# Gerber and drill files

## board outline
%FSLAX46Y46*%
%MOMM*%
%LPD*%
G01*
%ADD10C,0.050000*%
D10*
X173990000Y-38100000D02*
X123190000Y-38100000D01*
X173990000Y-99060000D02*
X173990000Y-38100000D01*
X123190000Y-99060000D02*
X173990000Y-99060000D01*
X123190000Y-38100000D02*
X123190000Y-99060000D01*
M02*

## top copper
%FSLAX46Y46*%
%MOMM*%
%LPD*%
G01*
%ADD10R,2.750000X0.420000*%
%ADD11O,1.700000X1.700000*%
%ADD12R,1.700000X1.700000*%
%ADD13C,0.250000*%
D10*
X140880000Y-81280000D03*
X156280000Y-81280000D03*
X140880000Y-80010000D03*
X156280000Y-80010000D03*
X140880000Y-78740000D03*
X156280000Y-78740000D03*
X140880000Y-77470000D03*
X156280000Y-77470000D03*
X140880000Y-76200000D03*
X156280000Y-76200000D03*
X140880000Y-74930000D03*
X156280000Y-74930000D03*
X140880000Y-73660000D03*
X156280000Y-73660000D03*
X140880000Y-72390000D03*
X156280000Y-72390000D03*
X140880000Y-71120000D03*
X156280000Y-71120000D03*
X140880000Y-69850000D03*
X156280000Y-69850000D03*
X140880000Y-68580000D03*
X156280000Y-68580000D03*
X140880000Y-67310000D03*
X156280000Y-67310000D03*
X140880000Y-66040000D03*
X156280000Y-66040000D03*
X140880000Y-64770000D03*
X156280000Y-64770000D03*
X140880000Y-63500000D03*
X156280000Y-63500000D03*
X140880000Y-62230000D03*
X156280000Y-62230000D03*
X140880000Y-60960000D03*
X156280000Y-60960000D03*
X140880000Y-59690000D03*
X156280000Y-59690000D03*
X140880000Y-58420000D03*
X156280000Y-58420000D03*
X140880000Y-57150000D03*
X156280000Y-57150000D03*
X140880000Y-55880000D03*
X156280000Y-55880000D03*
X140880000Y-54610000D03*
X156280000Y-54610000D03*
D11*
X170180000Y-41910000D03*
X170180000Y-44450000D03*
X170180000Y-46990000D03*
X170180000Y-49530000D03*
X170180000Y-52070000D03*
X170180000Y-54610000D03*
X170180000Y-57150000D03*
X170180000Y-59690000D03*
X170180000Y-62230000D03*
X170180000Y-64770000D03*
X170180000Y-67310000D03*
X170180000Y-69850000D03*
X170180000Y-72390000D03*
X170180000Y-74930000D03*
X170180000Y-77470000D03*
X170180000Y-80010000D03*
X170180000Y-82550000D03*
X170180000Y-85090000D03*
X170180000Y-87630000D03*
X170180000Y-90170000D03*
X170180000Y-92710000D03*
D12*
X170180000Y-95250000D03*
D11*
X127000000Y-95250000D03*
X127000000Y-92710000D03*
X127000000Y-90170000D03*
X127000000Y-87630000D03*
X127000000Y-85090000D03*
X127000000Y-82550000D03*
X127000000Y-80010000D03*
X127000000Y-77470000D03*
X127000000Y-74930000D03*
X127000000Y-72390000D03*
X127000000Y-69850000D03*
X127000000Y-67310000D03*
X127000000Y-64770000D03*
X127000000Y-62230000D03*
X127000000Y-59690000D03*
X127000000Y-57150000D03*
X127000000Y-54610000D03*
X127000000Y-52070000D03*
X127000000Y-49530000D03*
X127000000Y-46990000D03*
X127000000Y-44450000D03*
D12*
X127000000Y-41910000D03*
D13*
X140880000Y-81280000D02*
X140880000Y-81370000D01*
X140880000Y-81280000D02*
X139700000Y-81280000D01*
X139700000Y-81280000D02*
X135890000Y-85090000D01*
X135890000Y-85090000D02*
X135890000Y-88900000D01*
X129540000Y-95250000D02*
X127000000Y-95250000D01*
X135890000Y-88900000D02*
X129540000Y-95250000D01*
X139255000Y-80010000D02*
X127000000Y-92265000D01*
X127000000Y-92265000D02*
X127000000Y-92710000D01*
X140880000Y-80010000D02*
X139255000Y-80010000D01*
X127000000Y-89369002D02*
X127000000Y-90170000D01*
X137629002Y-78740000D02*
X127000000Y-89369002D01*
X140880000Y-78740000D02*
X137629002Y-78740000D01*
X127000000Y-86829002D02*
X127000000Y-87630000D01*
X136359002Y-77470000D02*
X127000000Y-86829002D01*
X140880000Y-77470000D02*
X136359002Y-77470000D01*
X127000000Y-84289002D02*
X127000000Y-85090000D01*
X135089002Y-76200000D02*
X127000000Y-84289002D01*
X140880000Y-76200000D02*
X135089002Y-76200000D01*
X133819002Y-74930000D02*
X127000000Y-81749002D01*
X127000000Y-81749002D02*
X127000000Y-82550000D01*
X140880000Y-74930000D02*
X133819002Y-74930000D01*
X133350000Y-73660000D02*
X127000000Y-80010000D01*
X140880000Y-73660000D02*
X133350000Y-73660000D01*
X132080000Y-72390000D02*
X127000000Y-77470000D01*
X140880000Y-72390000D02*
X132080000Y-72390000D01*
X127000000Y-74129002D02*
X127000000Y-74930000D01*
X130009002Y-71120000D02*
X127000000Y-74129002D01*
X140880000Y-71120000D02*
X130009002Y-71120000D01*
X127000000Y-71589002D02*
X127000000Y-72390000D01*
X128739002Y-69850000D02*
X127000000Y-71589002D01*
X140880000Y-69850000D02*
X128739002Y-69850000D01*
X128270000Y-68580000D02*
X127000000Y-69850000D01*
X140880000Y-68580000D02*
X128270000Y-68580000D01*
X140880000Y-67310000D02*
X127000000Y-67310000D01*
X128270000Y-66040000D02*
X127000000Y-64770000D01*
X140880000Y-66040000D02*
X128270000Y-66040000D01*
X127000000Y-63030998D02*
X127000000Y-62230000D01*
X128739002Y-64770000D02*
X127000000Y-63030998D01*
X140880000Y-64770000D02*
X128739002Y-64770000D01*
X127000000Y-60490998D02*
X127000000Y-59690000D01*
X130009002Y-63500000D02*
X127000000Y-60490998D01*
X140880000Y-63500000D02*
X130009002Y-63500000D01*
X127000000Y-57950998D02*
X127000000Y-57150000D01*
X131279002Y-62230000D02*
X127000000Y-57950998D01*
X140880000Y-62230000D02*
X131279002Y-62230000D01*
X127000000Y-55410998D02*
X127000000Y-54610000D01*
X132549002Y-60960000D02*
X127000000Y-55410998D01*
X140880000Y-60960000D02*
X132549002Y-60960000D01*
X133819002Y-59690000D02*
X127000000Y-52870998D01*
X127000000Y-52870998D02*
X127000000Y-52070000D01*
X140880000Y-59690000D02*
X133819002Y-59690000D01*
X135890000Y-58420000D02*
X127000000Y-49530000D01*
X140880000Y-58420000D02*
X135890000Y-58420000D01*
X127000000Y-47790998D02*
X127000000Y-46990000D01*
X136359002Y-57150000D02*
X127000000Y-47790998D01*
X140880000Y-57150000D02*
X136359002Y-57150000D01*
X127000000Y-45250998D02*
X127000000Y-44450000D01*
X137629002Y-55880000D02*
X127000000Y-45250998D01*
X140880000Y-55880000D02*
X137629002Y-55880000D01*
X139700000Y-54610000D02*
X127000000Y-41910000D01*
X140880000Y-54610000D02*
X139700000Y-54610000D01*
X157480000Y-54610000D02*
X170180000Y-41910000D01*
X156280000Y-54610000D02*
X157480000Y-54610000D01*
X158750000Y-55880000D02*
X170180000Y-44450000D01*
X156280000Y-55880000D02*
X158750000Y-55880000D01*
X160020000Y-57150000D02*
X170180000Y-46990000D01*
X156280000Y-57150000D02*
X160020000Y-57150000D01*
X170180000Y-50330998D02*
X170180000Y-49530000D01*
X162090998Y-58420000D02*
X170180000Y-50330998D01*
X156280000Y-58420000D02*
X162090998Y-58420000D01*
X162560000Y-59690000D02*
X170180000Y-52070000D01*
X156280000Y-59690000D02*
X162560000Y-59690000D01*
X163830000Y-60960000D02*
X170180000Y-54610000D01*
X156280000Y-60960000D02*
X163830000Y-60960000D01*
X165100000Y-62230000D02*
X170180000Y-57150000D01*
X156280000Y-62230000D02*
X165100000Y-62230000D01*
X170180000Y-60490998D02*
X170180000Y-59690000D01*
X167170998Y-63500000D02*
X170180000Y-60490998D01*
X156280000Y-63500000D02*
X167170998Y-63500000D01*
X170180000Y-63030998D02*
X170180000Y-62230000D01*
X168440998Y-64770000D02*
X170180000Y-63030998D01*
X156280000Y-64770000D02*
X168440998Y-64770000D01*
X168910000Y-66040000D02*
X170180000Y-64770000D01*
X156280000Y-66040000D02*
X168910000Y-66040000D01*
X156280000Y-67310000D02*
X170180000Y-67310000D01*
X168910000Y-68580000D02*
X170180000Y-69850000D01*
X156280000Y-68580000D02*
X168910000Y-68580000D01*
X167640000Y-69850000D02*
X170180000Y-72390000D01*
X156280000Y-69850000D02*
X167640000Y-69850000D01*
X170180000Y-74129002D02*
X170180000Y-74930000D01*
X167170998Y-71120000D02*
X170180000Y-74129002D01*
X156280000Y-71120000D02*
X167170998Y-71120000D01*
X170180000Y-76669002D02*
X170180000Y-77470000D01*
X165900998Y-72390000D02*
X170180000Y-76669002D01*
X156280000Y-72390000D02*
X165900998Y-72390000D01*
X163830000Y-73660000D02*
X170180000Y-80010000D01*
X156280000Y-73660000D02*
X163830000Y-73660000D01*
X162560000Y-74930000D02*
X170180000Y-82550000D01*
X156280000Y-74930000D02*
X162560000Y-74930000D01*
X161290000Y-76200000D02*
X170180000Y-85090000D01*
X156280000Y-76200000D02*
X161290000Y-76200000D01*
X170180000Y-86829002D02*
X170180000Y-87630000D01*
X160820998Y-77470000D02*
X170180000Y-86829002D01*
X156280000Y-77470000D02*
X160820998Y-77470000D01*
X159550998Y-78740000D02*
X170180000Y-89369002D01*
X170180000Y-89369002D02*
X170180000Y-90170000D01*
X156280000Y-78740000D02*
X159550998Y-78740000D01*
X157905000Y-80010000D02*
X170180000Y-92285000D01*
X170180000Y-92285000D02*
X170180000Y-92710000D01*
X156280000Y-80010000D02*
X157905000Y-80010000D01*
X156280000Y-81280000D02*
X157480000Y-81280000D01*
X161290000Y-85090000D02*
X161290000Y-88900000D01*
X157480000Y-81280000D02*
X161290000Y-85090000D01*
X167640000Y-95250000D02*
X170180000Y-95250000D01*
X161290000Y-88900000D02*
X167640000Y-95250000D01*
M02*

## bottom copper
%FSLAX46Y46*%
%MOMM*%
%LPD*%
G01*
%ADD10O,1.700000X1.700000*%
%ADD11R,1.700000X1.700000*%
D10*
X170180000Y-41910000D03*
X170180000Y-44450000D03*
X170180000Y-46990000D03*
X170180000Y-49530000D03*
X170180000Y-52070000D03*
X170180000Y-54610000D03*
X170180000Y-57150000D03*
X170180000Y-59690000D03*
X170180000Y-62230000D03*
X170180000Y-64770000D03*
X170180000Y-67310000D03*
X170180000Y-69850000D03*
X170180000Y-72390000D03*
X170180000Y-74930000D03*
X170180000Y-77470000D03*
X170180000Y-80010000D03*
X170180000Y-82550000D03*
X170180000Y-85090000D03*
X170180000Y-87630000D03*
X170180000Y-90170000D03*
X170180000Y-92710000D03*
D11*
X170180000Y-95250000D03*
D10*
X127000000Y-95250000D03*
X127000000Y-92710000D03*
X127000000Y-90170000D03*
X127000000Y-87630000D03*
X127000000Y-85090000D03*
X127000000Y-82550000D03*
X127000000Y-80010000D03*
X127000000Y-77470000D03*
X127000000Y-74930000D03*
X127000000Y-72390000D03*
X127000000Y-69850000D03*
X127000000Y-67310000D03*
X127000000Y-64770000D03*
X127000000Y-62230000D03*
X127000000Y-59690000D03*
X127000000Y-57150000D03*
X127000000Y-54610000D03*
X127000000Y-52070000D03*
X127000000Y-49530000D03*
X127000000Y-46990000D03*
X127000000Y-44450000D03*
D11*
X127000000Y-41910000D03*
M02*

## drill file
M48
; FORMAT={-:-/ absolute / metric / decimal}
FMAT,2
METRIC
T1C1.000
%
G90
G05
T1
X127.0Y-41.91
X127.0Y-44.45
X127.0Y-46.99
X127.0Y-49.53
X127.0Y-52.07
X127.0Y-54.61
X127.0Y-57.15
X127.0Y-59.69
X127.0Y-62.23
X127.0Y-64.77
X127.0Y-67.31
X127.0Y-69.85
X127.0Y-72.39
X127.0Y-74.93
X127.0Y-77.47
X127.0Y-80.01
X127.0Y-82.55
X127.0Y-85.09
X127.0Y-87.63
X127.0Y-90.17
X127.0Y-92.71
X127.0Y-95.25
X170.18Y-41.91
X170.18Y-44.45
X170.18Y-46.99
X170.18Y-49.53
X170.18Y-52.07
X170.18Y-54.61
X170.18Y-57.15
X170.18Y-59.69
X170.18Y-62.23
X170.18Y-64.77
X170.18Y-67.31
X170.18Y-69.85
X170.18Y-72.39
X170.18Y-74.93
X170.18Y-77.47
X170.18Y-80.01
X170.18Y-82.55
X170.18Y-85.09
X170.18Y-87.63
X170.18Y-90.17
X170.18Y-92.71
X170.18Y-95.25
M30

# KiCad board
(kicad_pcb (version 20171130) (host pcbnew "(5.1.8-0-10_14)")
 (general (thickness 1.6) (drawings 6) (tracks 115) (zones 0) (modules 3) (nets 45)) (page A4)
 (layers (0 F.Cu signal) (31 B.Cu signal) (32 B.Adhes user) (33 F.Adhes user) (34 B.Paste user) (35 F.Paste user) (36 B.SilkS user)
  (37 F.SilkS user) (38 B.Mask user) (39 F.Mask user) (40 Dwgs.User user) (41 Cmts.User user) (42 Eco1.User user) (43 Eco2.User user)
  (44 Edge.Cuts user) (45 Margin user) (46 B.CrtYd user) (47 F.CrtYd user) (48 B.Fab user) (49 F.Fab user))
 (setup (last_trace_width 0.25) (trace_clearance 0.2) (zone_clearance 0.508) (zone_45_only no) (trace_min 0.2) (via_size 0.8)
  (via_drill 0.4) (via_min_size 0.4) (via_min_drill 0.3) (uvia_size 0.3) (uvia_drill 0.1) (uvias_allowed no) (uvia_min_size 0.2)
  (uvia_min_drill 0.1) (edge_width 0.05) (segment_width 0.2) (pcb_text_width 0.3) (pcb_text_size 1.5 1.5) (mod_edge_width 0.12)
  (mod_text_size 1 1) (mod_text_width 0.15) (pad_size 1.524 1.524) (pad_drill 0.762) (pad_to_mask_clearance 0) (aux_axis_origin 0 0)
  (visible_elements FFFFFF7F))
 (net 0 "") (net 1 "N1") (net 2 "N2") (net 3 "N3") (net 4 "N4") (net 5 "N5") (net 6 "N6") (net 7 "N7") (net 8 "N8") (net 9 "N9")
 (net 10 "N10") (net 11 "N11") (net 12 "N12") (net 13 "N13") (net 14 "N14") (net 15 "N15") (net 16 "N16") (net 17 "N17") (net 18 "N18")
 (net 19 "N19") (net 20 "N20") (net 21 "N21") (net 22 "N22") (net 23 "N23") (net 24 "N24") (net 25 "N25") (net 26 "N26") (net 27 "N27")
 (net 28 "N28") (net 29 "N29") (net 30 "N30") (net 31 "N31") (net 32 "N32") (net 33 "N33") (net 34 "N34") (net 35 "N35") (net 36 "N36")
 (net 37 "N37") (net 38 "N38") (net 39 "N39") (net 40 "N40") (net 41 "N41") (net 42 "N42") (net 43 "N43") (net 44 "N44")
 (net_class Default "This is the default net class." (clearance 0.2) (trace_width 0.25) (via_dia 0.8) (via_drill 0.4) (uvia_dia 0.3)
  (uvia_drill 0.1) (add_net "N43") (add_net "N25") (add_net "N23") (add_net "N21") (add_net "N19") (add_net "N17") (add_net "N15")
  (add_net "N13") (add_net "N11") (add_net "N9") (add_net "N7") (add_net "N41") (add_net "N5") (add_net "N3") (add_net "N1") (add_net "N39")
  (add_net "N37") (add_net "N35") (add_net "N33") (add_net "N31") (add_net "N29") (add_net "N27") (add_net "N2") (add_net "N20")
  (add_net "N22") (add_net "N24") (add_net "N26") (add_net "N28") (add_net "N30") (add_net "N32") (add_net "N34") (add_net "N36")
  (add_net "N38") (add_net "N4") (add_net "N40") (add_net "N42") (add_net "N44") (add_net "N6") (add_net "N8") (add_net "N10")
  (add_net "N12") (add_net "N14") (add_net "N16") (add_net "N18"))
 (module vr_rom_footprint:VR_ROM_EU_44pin (layer F.Cu) (at 148.58 67.945 270)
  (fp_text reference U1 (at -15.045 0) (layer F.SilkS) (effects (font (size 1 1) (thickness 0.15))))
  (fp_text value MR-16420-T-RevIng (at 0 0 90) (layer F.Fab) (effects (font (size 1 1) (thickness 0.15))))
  (pad 22 smd rect (at 13.335 7.7 270) (size 0.42 2.75) (layers F.Cu F.Paste F.Mask) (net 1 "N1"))
  (pad 23 smd rect (at 13.335 -7.7 270) (size 0.42 2.75) (layers F.Cu F.Paste F.Mask) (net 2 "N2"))
  (pad 21 smd rect (at 12.065 7.7 270) (size 0.42 2.75) (layers F.Cu F.Paste F.Mask) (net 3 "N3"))
  (pad 24 smd rect (at 12.065 -7.7 270) (size 0.42 2.75) (layers F.Cu F.Paste F.Mask) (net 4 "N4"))
  (pad 20 smd rect (at 10.795 7.7 270) (size 0.42 2.75) (layers F.Cu F.Paste F.Mask) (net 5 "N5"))
  (pad 25 smd rect (at 10.795 -7.7 270) (size 0.42 2.75) (layers F.Cu F.Paste F.Mask) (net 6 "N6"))
  (pad 19 smd rect (at 9.525 7.7 270) (size 0.42 2.75) (layers F.Cu F.Paste F.Mask) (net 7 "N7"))
  (pad 26 smd rect (at 9.525 -7.7 270) (size 0.42 2.75) (layers F.Cu F.Paste F.Mask) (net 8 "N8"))
  (pad 18 smd rect (at 8.255 7.7 270) (size 0.42 2.75) (layers F.Cu F.Paste F.Mask) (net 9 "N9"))
  (pad 27 smd rect (at 8.255 -7.7 270) (size 0.42 2.75) (layers F.Cu F.Paste F.Mask) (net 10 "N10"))
  (pad 17 smd rect (at 6.985 7.7 270) (size 0.42 2.75) (layers F.Cu F.Paste F.Mask) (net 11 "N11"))
  (pad 28 smd rect (at 6.985 -7.7 270) (size 0.42 2.75) (layers F.Cu F.Paste F.Mask) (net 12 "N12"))
  (pad 16 smd rect (at 5.715 7.7 270) (size 0.42 2.75) (layers F.Cu F.Paste F.Mask) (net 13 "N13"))
  (pad 29 smd rect (at 5.715 -7.7 270) (size 0.42 2.75) (layers F.Cu F.Paste F.Mask) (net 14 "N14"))
  (pad 15 smd rect (at 4.445 7.7 270) (size 0.42 2.75) (layers F.Cu F.Paste F.Mask) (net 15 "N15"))
  (pad 30 smd rect (at 4.445 -7.7 270) (size 0.42 2.75) (layers F.Cu F.Paste F.Mask) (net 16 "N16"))
  (pad 14 smd rect (at 3.175 7.7 270) (size 0.42 2.75) (layers F.Cu F.Paste F.Mask) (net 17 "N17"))
  (pad 31 smd rect (at 3.175 -7.7 270) (size 0.42 2.75) (layers F.Cu F.Paste F.Mask) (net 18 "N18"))
  (pad 13 smd rect (at 1.905 7.7 270) (size 0.42 2.75) (layers F.Cu F.Paste F.Mask) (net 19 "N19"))
  (pad 32 smd rect (at 1.905 -7.7 270) (size 0.42 2.75) (layers F.Cu F.Paste F.Mask) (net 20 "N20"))
  (pad 12 smd rect (at 0.635 7.7 270) (size 0.42 2.75) (layers F.Cu F.Paste F.Mask) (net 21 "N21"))
  (pad 33 smd rect (at 0.635 -7.7 270) (size 0.42 2.75) (layers F.Cu F.Paste F.Mask) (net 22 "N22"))
  (pad 11 smd rect (at -0.635 7.7 270) (size 0.42 2.75) (layers F.Cu F.Paste F.Mask) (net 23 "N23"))
  (pad 34 smd rect (at -0.635 -7.7 270) (size 0.42 2.75) (layers F.Cu F.Paste F.Mask) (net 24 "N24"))
  (pad 10 smd rect (at -1.905 7.7 270) (size 0.42 2.75) (layers F.Cu F.Paste F.Mask) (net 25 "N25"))
  (pad 35 smd rect (at -1.905 -7.7 270) (size 0.42 2.75) (layers F.Cu F.Paste F.Mask) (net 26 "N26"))
  (pad 9 smd rect (at -3.175 7.7 270) (size 0.42 2.75) (layers F.Cu F.Paste F.Mask) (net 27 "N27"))
  (pad 36 smd rect (at -3.175 -7.7 270) (size 0.42 2.75) (layers F.Cu F.Paste F.Mask) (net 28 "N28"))
  (pad 8 smd rect (at -4.445 7.7 270) (size 0.42 2.75) (layers F.Cu F.Paste F.Mask) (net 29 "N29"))
  (pad 37 smd rect (at -4.445 -7.7 270) (size 0.42 2.75) (layers F.Cu F.Paste F.Mask) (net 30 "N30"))
  (pad 7 smd rect (at -5.715 7.7 270) (size 0.42 2.75) (layers F.Cu F.Paste F.Mask) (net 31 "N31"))
  (pad 38 smd rect (at -5.715 -7.7 270) (size 0.42 2.75) (layers F.Cu F.Paste F.Mask) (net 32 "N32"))
  (pad 6 smd rect (at -6.985 7.7 270) (size 0.42 2.75) (layers F.Cu F.Paste F.Mask) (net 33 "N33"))
  (pad 39 smd rect (at -6.985 -7.7 270) (size 0.42 2.75) (layers F.Cu F.Paste F.Mask) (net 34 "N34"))
  (pad 5 smd rect (at -8.255 7.7 270) (size 0.42 2.75) (layers F.Cu F.Paste F.Mask) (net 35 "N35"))
  (pad 40 smd rect (at -8.255 -7.7 270) (size 0.42 2.75) (layers F.Cu F.Paste F.Mask) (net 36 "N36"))
  (pad 4 smd rect (at -9.525 7.7 270) (size 0.42 2.75) (layers F.Cu F.Paste F.Mask) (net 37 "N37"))
  (pad 41 smd rect (at -9.525 -7.7 270) (size 0.42 2.75) (layers F.Cu F.Paste F.Mask) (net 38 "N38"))
  (pad 3 smd rect (at -10.795 7.7 270) (size 0.42 2.75) (layers F.Cu F.Paste F.Mask) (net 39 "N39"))
  (pad 42 smd rect (at -10.795 -7.7 270) (size 0.42 2.75) (layers F.Cu F.Paste F.Mask) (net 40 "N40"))
  (pad 2 smd rect (at -12.065 7.7 270) (size 0.42 2.75) (layers F.Cu F.Paste F.Mask) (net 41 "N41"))
  (pad 43 smd rect (at -12.065 -7.7 270) (size 0.42 2.75) (layers F.Cu F.Paste F.Mask) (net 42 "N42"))
  (pad 1 smd rect (at -13.335 7.7 270) (size 0.42 2.75) (layers F.Cu F.Paste F.Mask) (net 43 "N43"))
  (pad 44 smd rect (at -13.335 -7.7 270) (size 0.42 2.75) (layers F.Cu F.Paste F.Mask) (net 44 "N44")))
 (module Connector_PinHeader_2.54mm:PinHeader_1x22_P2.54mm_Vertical (layer F.Cu) (at 170.18 95.25 180)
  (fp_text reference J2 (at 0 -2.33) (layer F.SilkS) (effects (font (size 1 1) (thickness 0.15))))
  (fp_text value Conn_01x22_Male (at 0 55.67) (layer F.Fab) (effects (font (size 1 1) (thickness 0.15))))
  (pad 22 thru_hole oval (at 0 53.34 180) (size 1.7 1.7) (drill 1) (layers *.Cu *.Mask) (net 44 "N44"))
  (pad 21 thru_hole oval (at 0 50.8 180) (size 1.7 1.7) (drill 1) (layers *.Cu *.Mask) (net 42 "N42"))
  (pad 20 thru_hole oval (at 0 48.26 180) (size 1.7 1.7) (drill 1) (layers *.Cu *.Mask) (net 40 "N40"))
  (pad 19 thru_hole oval (at 0 45.72 180) (size 1.7 1.7) (drill 1) (layers *.Cu *.Mask) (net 38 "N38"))
  (pad 18 thru_hole oval (at 0 43.18 180) (size 1.7 1.7) (drill 1) (layers *.Cu *.Mask) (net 36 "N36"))
  (pad 17 thru_hole oval (at 0 40.64 180) (size 1.7 1.7) (drill 1) (layers *.Cu *.Mask) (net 34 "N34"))
  (pad 16 thru_hole oval (at 0 38.1 180) (size 1.7 1.7) (drill 1) (layers *.Cu *.Mask) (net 32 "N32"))
  (pad 15 thru_hole oval (at 0 35.56 180) (size 1.7 1.7) (drill 1) (layers *.Cu *.Mask) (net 30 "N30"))
  (pad 14 thru_hole oval (at 0 33.02 180) (size 1.7 1.7) (drill 1) (layers *.Cu *.Mask) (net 28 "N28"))
  (pad 13 thru_hole oval (at 0 30.48 180) (size 1.7 1.7) (drill 1) (layers *.Cu *.Mask) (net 26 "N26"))
  (pad 12 thru_hole oval (at 0 27.94 180) (size 1.7 1.7) (drill 1) (layers *.Cu *.Mask) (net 24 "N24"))
  (pad 11 thru_hole oval (at 0 25.4 180) (size 1.7 1.7) (drill 1) (layers *.Cu *.Mask) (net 22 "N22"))
  (pad 10 thru_hole oval (at 0 22.86 180) (size 1.7 1.7) (drill 1) (layers *.Cu *.Mask) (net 20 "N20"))
  (pad 9 thru_hole oval (at 0 20.32 180) (size 1.7 1.7) (drill 1) (layers *.Cu *.Mask) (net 18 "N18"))
  (pad 8 thru_hole oval (at 0 17.78 180) (size 1.7 1.7) (drill 1) (layers *.Cu *.Mask) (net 16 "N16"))
  (pad 7 thru_hole oval (at 0 15.24 180) (size 1.7 1.7) (drill 1) (layers *.Cu *.Mask) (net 14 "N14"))
  (pad 6 thru_hole oval (at 0 12.7 180) (size 1.7 1.7) (drill 1) (layers *.Cu *.Mask) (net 12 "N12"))
  (pad 5 thru_hole oval (at 0 10.16 180) (size 1.7 1.7) (drill 1) (layers *.Cu *.Mask) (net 10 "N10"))
  (pad 4 thru_hole oval (at 0 7.62 180) (size 1.7 1.7) (drill 1) (layers *.Cu *.Mask) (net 8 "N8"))
  (pad 3 thru_hole oval (at 0 5.08 180) (size 1.7 1.7) (drill 1) (layers *.Cu *.Mask) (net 6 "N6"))
  (pad 2 thru_hole oval (at 0 2.54 180) (size 1.7 1.7) (drill 1) (layers *.Cu *.Mask) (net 4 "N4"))
  (pad 1 thru_hole rect (at 0 0 180) (size 1.7 1.7) (drill 1) (layers *.Cu *.Mask) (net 2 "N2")))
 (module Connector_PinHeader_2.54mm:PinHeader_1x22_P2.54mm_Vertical (layer F.Cu) (at 127 41.91)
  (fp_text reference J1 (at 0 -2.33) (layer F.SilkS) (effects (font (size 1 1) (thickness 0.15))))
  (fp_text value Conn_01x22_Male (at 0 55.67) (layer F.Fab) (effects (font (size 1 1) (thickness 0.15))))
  (pad 22 thru_hole oval (at 0 53.34) (size 1.7 1.7) (drill 1) (layers *.Cu *.Mask) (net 1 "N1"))
  (pad 21 thru_hole oval (at 0 50.8) (size 1.7 1.7) (drill 1) (layers *.Cu *.Mask) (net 3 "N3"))
  (pad 20 thru_hole oval (at 0 48.26) (size 1.7 1.7) (drill 1) (layers *.Cu *.Mask) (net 5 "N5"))
  (pad 19 thru_hole oval (at 0 45.72) (size 1.7 1.7) (drill 1) (layers *.Cu *.Mask) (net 7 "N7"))
  (pad 18 thru_hole oval (at 0 43.18) (size 1.7 1.7) (drill 1) (layers *.Cu *.Mask) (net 9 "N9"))
  (pad 17 thru_hole oval (at 0 40.64) (size 1.7 1.7) (drill 1) (layers *.Cu *.Mask) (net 11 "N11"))
  (pad 16 thru_hole oval (at 0 38.1) (size 1.7 1.7) (drill 1) (layers *.Cu *.Mask) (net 13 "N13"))
  (pad 15 thru_hole oval (at 0 35.56) (size 1.7 1.7) (drill 1) (layers *.Cu *.Mask) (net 15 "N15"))
  (pad 14 thru_hole oval (at 0 33.02) (size 1.7 1.7) (drill 1) (layers *.Cu *.Mask) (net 17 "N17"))
  (pad 13 thru_hole oval (at 0 30.48) (size 1.7 1.7) (drill 1) (layers *.Cu *.Mask) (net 19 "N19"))
  (pad 12 thru_hole oval (at 0 27.94) (size 1.7 1.7) (drill 1) (layers *.Cu *.Mask) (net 21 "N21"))
  (pad 11 thru_hole oval (at 0 25.4) (size 1.7 1.7) (drill 1) (layers *.Cu *.Mask) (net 23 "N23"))
  (pad 10 thru_hole oval (at 0 22.86) (size 1.7 1.7) (drill 1) (layers *.Cu *.Mask) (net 25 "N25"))
  (pad 9 thru_hole oval (at 0 20.32) (size 1.7 1.7) (drill 1) (layers *.Cu *.Mask) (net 27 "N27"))
  (pad 8 thru_hole oval (at 0 17.78) (size 1.7 1.7) (drill 1) (layers *.Cu *.Mask) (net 29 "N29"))
  (pad 7 thru_hole oval (at 0 15.24) (size 1.7 1.7) (drill 1) (layers *.Cu *.Mask) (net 31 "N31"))
  (pad 6 thru_hole oval (at 0 12.7) (size 1.7 1.7) (drill 1) (layers *.Cu *.Mask) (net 33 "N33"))
  (pad 5 thru_hole oval (at 0 10.16) (size 1.7 1.7) (drill 1) (layers *.Cu *.Mask) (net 35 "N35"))
  (pad 4 thru_hole oval (at 0 7.62) (size 1.7 1.7) (drill 1) (layers *.Cu *.Mask) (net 37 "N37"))
  (pad 3 thru_hole oval (at 0 5.08) (size 1.7 1.7) (drill 1) (layers *.Cu *.Mask) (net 39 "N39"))
  (pad 2 thru_hole oval (at 0 2.54) (size 1.7 1.7) (drill 1) (layers *.Cu *.Mask) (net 41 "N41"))
  (pad 1 thru_hole rect (at 0 0) (size 1.7 1.7) (drill 1) (layers *.Cu *.Mask) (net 43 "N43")))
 (gr_line (start 173.99 38.1) (end 123.19 38.1) (layer Edge.Cuts) (width 0.05))
 (gr_line (start 173.99 99.06) (end 173.99 38.1) (layer Edge.Cuts) (width 0.05))
 (gr_line (start 123.19 99.06) (end 173.99 99.06) (layer Edge.Cuts) (width 0.05))
 (gr_line (start 123.19 38.1) (end 123.19 99.06) (layer Edge.Cuts) (width 0.05))
 (segment (start 140.88 81.28) (end 140.88 81.37) (width 0.25) (layer F.Cu) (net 1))
 (segment (start 140.88 81.28) (end 139.7 81.28) (width 0.25) (layer F.Cu) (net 1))
 (segment (start 139.7 81.28) (end 135.89 85.09) (width 0.25) (layer F.Cu) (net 1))
 (segment (start 135.89 85.09) (end 135.89 88.9) (width 0.25) (layer F.Cu) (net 1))
 (segment (start 129.54 95.25) (end 127 95.25) (width 0.25) (layer F.Cu) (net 1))
 (segment (start 135.89 88.9) (end 129.54 95.25) (width 0.25) (layer F.Cu) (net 1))
 (segment (start 139.255 80.01) (end 127 92.265) (width 0.25) (layer F.Cu) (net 3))
 (segment (start 127 92.265) (end 127 92.71) (width 0.25) (layer F.Cu) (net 3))
 (segment (start 140.88 80.01) (end 139.255 80.01) (width 0.25) (layer F.Cu) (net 3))
 (segment (start 127 89.369002) (end 127 90.17) (width 0.25) (layer F.Cu) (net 5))
 (segment (start 137.629002 78.74) (end 127 89.369002) (width 0.25) (layer F.Cu) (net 5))
 (segment (start 140.88 78.74) (end 137.629002 78.74) (width 0.25) (layer F.Cu) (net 5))
 (segment (start 127 86.829002) (end 127 87.63) (width 0.25) (layer F.Cu) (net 7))
 (segment (start 136.359002 77.47) (end 127 86.829002) (width 0.25) (layer F.Cu) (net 7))
 (segment (start 140.88 77.47) (end 136.359002 77.47) (width 0.25) (layer F.Cu) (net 7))
 (segment (start 127 84.289002) (end 127 85.09) (width 0.25) (layer F.Cu) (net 9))
 (segment (start 135.089002 76.2) (end 127 84.289002) (width 0.25) (layer F.Cu) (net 9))
 (segment (start 140.88 76.2) (end 135.089002 76.2) (width 0.25) (layer F.Cu) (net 9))
 (segment (start 133.819002 74.93) (end 127 81.749002) (width 0.25) (layer F.Cu) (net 11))
 (segment (start 127 81.749002) (end 127 82.55) (width 0.25) (layer F.Cu) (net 11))
 (segment (start 140.88 74.93) (end 133.819002 74.93) (width 0.25) (layer F.Cu) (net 11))
 (segment (start 133.35 73.66) (end 127 80.01) (width 0.25) (layer F.Cu) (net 13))
 (segment (start 140.88 73.66) (end 133.35 73.66) (width 0.25) (layer F.Cu) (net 13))
 (segment (start 132.08 72.39) (end 127 77.47) (width 0.25) (layer F.Cu) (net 15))
 (segment (start 140.88 72.39) (end 132.08 72.39) (width 0.25) (layer F.Cu) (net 15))
 (segment (start 127 74.129002) (end 127 74.93) (width 0.25) (layer F.Cu) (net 17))
 (segment (start 130.009002 71.12) (end 127 74.129002) (width 0.25) (layer F.Cu) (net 17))
 (segment (start 140.88 71.12) (end 130.009002 71.12) (width 0.25) (layer F.Cu) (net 17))
 (segment (start 127 71.589002) (end 127 72.39) (width 0.25) (layer F.Cu) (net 19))
 (segment (start 128.739002 69.85) (end 127 71.589002) (width 0.25) (layer F.Cu) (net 19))
 (segment (start 140.88 69.85) (end 128.739002 69.85) (width 0.25) (layer F.Cu) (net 19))
 (segment (start 128.27 68.58) (end 127 69.85) (width 0.25) (layer F.Cu) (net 21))
 (segment (start 140.88 68.58) (end 128.27 68.58) (width 0.25) (layer F.Cu) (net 21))
 (segment (start 140.88 67.31) (end 127 67.31) (width 0.25) (layer F.Cu) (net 23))
 (segment (start 128.27 66.04) (end 127 64.77) (width 0.25) (layer F.Cu) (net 25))
 (segment (start 140.88 66.04) (end 128.27 66.04) (width 0.25) (layer F.Cu) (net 25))
 (segment (start 127 63.030998) (end 127 62.23) (width 0.25) (layer F.Cu) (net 27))
 (segment (start 128.739002 64.77) (end 127 63.030998) (width 0.25) (layer F.Cu) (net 27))
 (segment (start 140.88 64.77) (end 128.739002 64.77) (width 0.25) (layer F.Cu) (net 27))
 (segment (start 127 60.490998) (end 127 59.69) (width 0.25) (layer F.Cu) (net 29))
 (segment (start 130.009002 63.5) (end 127 60.490998) (width 0.25) (layer F.Cu) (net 29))
 (segment (start 140.88 63.5) (end 130.009002 63.5) (width 0.25) (layer F.Cu) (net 29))
 (segment (start 127 57.950998) (end 127 57.15) (width 0.25) (layer F.Cu) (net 31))
 (segment (start 131.279002 62.23) (end 127 57.950998) (width 0.25) (layer F.Cu) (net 31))
 (segment (start 140.88 62.23) (end 131.279002 62.23) (width 0.25) (layer F.Cu) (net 31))
 (segment (start 127 55.410998) (end 127 54.61) (width 0.25) (layer F.Cu) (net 33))
 (segment (start 132.549002 60.96) (end 127 55.410998) (width 0.25) (layer F.Cu) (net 33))
 (segment (start 140.88 60.96) (end 132.549002 60.96) (width 0.25) (layer F.Cu) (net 33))
 (segment (start 133.819002 59.69) (end 127 52.870998) (width 0.25) (layer F.Cu) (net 35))
 (segment (start 127 52.870998) (end 127 52.07) (width 0.25) (layer F.Cu) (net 35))
 (segment (start 140.88 59.69) (end 133.819002 59.69) (width 0.25) (layer F.Cu) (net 35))
 (segment (start 135.89 58.42) (end 127 49.53) (width 0.25) (layer F.Cu) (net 37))
 (segment (start 140.88 58.42) (end 135.89 58.42) (width 0.25) (layer F.Cu) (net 37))
 (segment (start 127 47.790998) (end 127 46.99) (width 0.25) (layer F.Cu) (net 39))
 (segment (start 136.359002 57.15) (end 127 47.790998) (width 0.25) (layer F.Cu) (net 39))
 (segment (start 140.88 57.15) (end 136.359002 57.15) (width 0.25) (layer F.Cu) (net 39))
 (segment (start 127 45.250998) (end 127 44.45) (width 0.25) (layer F.Cu) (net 41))
 (segment (start 137.629002 55.88) (end 127 45.250998) (width 0.25) (layer F.Cu) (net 41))
 (segment (start 140.88 55.88) (end 137.629002 55.88) (width 0.25) (layer F.Cu) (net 41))
 (segment (start 139.7 54.61) (end 127 41.91) (width 0.25) (layer F.Cu) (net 43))
 (segment (start 140.88 54.61) (end 139.7 54.61) (width 0.25) (layer F.Cu) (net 43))
 (segment (start 157.48 54.61) (end 170.18 41.91) (width 0.25) (layer F.Cu) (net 44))
 (segment (start 156.28 54.61) (end 157.48 54.61) (width 0.25) (layer F.Cu) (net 44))
 (segment (start 158.75 55.88) (end 170.18 44.45) (width 0.25) (layer F.Cu) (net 42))
 (segment (start 156.28 55.88) (end 158.75 55.88) (width 0.25) (layer F.Cu) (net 42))
 (segment (start 160.02 57.15) (end 170.18 46.99) (width 0.25) (layer F.Cu) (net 40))
 (segment (start 156.28 57.15) (end 160.02 57.15) (width 0.25) (layer F.Cu) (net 40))
 (segment (start 170.18 50.330998) (end 170.18 49.53) (width 0.25) (layer F.Cu) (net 38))
 (segment (start 162.090998 58.42) (end 170.18 50.330998) (width 0.25) (layer F.Cu) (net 38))
 (segment (start 156.28 58.42) (end 162.090998 58.42) (width 0.25) (layer F.Cu) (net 38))
 (segment (start 162.56 59.69) (end 170.18 52.07) (width 0.25) (layer F.Cu) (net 36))
 (segment (start 156.28 59.69) (end 162.56 59.69) (width 0.25) (layer F.Cu) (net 36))
 (segment (start 163.83 60.96) (end 170.18 54.61) (width 0.25) (layer F.Cu) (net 34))
 (segment (start 156.28 60.96) (end 163.83 60.96) (width 0.25) (layer F.Cu) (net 34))
 (segment (start 165.1 62.23) (end 170.18 57.15) (width 0.25) (layer F.Cu) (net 32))
 (segment (start 156.28 62.23) (end 165.1 62.23) (width 0.25) (layer F.Cu) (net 32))
 (segment (start 170.18 60.490998) (end 170.18 59.69) (width 0.25) (layer F.Cu) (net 30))
 (segment (start 167.170998 63.5) (end 170.18 60.490998) (width 0.25) (layer F.Cu) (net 30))
 (segment (start 156.28 63.5) (end 167.170998 63.5) (width 0.25) (layer F.Cu) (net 30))
 (segment (start 170.18 63.030998) (end 170.18 62.23) (width 0.25) (layer F.Cu) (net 28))
 (segment (start 168.440998 64.77) (end 170.18 63.030998) (width 0.25) (layer F.Cu) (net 28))
 (segment (start 156.28 64.77) (end 168.440998 64.77) (width 0.25) (layer F.Cu) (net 28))
 (segment (start 168.91 66.04) (end 170.18 64.77) (width 0.25) (layer F.Cu) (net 26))
 (segment (start 156.28 66.04) (end 168.91 66.04) (width 0.25) (layer F.Cu) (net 26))
 (segment (start 156.28 67.31) (end 170.18 67.31) (width 0.25) (layer F.Cu) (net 24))
 (segment (start 168.91 68.58) (end 170.18 69.85) (width 0.25) (layer F.Cu) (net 22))
 (segment (start 156.28 68.58) (end 168.91 68.58) (width 0.25) (layer F.Cu) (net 22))
 (segment (start 167.64 69.85) (end 170.18 72.39) (width 0.25) (layer F.Cu) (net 20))
 (segment (start 156.28 69.85) (end 167.64 69.85) (width 0.25) (layer F.Cu) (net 20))
 (segment (start 170.18 74.129002) (end 170.18 74.93) (width 0.25) (layer F.Cu) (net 18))
 (segment (start 167.170998 71.12) (end 170.18 74.129002) (width 0.25) (layer F.Cu) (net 18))
 (segment (start 156.28 71.12) (end 167.170998 71.12) (width 0.25) (layer F.Cu) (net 18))
 (segment (start 170.18 76.669002) (end 170.18 77.47) (width 0.25) (layer F.Cu) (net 16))
 (segment (start 165.900998 72.39) (end 170.18 76.669002) (width 0.25) (layer F.Cu) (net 16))
 (segment (start 156.28 72.39) (end 165.900998 72.39) (width 0.25) (layer F.Cu) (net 16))
 (segment (start 163.83 73.66) (end 170.18 80.01) (width 0.25) (layer F.Cu) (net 14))
 (segment (start 156.28 73.66) (end 163.83 73.66) (width 0.25) (layer F.Cu) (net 14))
 (segment (start 162.56 74.93) (end 170.18 82.55) (width 0.25) (layer F.Cu) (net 12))
 (segment (start 156.28 74.93) (end 162.56 74.93) (width 0.25) (layer F.Cu) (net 12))
 (segment (start 161.29 76.2) (end 170.18 85.09) (width 0.25) (layer F.Cu) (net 10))
 (segment (start 156.28 76.2) (end 161.29 76.2) (width 0.25) (layer F.Cu) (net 10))
 (segment (start 170.18 86.829002) (end 170.18 87.63) (width 0.25) (layer F.Cu) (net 8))
 (segment (start 160.820998 77.47) (end 170.18 86.829002) (width 0.25) (layer F.Cu) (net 8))
 (segment (start 156.28 77.47) (end 160.820998 77.47) (width 0.25) (layer F.Cu) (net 8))
 (segment (start 159.550998 78.74) (end 170.18 89.369002) (width 0.25) (layer F.Cu) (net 6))
 (segment (start 170.18 89.369002) (end 170.18 90.17) (width 0.25) (layer F.Cu) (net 6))
 (segment (start 156.28 78.74) (end 159.550998 78.74) (width 0.25) (layer F.Cu) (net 6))
 (segment (start 157.905 80.01) (end 170.18 92.285) (width 0.25) (layer F.Cu) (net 4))
 (segment (start 170.18 92.285) (end 170.18 92.71) (width 0.25) (layer F.Cu) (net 4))
 (segment (start 156.28 80.01) (end 157.905 80.01) (width 0.25) (layer F.Cu) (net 4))
 (segment (start 156.28 81.28) (end 157.48 81.28) (width 0.25) (layer F.Cu) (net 2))
 (segment (start 161.29 85.09) (end 161.29 88.9) (width 0.25) (layer F.Cu) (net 2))
 (segment (start 157.48 81.28) (end 161.29 85.09) (width 0.25) (layer F.Cu) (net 2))
 (segment (start 167.64 95.25) (end 170.18 95.25) (width 0.25) (layer F.Cu) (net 2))
 (segment (start 161.29 88.9) (end 167.64 95.25) (width 0.25) (layer F.Cu) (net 2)))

